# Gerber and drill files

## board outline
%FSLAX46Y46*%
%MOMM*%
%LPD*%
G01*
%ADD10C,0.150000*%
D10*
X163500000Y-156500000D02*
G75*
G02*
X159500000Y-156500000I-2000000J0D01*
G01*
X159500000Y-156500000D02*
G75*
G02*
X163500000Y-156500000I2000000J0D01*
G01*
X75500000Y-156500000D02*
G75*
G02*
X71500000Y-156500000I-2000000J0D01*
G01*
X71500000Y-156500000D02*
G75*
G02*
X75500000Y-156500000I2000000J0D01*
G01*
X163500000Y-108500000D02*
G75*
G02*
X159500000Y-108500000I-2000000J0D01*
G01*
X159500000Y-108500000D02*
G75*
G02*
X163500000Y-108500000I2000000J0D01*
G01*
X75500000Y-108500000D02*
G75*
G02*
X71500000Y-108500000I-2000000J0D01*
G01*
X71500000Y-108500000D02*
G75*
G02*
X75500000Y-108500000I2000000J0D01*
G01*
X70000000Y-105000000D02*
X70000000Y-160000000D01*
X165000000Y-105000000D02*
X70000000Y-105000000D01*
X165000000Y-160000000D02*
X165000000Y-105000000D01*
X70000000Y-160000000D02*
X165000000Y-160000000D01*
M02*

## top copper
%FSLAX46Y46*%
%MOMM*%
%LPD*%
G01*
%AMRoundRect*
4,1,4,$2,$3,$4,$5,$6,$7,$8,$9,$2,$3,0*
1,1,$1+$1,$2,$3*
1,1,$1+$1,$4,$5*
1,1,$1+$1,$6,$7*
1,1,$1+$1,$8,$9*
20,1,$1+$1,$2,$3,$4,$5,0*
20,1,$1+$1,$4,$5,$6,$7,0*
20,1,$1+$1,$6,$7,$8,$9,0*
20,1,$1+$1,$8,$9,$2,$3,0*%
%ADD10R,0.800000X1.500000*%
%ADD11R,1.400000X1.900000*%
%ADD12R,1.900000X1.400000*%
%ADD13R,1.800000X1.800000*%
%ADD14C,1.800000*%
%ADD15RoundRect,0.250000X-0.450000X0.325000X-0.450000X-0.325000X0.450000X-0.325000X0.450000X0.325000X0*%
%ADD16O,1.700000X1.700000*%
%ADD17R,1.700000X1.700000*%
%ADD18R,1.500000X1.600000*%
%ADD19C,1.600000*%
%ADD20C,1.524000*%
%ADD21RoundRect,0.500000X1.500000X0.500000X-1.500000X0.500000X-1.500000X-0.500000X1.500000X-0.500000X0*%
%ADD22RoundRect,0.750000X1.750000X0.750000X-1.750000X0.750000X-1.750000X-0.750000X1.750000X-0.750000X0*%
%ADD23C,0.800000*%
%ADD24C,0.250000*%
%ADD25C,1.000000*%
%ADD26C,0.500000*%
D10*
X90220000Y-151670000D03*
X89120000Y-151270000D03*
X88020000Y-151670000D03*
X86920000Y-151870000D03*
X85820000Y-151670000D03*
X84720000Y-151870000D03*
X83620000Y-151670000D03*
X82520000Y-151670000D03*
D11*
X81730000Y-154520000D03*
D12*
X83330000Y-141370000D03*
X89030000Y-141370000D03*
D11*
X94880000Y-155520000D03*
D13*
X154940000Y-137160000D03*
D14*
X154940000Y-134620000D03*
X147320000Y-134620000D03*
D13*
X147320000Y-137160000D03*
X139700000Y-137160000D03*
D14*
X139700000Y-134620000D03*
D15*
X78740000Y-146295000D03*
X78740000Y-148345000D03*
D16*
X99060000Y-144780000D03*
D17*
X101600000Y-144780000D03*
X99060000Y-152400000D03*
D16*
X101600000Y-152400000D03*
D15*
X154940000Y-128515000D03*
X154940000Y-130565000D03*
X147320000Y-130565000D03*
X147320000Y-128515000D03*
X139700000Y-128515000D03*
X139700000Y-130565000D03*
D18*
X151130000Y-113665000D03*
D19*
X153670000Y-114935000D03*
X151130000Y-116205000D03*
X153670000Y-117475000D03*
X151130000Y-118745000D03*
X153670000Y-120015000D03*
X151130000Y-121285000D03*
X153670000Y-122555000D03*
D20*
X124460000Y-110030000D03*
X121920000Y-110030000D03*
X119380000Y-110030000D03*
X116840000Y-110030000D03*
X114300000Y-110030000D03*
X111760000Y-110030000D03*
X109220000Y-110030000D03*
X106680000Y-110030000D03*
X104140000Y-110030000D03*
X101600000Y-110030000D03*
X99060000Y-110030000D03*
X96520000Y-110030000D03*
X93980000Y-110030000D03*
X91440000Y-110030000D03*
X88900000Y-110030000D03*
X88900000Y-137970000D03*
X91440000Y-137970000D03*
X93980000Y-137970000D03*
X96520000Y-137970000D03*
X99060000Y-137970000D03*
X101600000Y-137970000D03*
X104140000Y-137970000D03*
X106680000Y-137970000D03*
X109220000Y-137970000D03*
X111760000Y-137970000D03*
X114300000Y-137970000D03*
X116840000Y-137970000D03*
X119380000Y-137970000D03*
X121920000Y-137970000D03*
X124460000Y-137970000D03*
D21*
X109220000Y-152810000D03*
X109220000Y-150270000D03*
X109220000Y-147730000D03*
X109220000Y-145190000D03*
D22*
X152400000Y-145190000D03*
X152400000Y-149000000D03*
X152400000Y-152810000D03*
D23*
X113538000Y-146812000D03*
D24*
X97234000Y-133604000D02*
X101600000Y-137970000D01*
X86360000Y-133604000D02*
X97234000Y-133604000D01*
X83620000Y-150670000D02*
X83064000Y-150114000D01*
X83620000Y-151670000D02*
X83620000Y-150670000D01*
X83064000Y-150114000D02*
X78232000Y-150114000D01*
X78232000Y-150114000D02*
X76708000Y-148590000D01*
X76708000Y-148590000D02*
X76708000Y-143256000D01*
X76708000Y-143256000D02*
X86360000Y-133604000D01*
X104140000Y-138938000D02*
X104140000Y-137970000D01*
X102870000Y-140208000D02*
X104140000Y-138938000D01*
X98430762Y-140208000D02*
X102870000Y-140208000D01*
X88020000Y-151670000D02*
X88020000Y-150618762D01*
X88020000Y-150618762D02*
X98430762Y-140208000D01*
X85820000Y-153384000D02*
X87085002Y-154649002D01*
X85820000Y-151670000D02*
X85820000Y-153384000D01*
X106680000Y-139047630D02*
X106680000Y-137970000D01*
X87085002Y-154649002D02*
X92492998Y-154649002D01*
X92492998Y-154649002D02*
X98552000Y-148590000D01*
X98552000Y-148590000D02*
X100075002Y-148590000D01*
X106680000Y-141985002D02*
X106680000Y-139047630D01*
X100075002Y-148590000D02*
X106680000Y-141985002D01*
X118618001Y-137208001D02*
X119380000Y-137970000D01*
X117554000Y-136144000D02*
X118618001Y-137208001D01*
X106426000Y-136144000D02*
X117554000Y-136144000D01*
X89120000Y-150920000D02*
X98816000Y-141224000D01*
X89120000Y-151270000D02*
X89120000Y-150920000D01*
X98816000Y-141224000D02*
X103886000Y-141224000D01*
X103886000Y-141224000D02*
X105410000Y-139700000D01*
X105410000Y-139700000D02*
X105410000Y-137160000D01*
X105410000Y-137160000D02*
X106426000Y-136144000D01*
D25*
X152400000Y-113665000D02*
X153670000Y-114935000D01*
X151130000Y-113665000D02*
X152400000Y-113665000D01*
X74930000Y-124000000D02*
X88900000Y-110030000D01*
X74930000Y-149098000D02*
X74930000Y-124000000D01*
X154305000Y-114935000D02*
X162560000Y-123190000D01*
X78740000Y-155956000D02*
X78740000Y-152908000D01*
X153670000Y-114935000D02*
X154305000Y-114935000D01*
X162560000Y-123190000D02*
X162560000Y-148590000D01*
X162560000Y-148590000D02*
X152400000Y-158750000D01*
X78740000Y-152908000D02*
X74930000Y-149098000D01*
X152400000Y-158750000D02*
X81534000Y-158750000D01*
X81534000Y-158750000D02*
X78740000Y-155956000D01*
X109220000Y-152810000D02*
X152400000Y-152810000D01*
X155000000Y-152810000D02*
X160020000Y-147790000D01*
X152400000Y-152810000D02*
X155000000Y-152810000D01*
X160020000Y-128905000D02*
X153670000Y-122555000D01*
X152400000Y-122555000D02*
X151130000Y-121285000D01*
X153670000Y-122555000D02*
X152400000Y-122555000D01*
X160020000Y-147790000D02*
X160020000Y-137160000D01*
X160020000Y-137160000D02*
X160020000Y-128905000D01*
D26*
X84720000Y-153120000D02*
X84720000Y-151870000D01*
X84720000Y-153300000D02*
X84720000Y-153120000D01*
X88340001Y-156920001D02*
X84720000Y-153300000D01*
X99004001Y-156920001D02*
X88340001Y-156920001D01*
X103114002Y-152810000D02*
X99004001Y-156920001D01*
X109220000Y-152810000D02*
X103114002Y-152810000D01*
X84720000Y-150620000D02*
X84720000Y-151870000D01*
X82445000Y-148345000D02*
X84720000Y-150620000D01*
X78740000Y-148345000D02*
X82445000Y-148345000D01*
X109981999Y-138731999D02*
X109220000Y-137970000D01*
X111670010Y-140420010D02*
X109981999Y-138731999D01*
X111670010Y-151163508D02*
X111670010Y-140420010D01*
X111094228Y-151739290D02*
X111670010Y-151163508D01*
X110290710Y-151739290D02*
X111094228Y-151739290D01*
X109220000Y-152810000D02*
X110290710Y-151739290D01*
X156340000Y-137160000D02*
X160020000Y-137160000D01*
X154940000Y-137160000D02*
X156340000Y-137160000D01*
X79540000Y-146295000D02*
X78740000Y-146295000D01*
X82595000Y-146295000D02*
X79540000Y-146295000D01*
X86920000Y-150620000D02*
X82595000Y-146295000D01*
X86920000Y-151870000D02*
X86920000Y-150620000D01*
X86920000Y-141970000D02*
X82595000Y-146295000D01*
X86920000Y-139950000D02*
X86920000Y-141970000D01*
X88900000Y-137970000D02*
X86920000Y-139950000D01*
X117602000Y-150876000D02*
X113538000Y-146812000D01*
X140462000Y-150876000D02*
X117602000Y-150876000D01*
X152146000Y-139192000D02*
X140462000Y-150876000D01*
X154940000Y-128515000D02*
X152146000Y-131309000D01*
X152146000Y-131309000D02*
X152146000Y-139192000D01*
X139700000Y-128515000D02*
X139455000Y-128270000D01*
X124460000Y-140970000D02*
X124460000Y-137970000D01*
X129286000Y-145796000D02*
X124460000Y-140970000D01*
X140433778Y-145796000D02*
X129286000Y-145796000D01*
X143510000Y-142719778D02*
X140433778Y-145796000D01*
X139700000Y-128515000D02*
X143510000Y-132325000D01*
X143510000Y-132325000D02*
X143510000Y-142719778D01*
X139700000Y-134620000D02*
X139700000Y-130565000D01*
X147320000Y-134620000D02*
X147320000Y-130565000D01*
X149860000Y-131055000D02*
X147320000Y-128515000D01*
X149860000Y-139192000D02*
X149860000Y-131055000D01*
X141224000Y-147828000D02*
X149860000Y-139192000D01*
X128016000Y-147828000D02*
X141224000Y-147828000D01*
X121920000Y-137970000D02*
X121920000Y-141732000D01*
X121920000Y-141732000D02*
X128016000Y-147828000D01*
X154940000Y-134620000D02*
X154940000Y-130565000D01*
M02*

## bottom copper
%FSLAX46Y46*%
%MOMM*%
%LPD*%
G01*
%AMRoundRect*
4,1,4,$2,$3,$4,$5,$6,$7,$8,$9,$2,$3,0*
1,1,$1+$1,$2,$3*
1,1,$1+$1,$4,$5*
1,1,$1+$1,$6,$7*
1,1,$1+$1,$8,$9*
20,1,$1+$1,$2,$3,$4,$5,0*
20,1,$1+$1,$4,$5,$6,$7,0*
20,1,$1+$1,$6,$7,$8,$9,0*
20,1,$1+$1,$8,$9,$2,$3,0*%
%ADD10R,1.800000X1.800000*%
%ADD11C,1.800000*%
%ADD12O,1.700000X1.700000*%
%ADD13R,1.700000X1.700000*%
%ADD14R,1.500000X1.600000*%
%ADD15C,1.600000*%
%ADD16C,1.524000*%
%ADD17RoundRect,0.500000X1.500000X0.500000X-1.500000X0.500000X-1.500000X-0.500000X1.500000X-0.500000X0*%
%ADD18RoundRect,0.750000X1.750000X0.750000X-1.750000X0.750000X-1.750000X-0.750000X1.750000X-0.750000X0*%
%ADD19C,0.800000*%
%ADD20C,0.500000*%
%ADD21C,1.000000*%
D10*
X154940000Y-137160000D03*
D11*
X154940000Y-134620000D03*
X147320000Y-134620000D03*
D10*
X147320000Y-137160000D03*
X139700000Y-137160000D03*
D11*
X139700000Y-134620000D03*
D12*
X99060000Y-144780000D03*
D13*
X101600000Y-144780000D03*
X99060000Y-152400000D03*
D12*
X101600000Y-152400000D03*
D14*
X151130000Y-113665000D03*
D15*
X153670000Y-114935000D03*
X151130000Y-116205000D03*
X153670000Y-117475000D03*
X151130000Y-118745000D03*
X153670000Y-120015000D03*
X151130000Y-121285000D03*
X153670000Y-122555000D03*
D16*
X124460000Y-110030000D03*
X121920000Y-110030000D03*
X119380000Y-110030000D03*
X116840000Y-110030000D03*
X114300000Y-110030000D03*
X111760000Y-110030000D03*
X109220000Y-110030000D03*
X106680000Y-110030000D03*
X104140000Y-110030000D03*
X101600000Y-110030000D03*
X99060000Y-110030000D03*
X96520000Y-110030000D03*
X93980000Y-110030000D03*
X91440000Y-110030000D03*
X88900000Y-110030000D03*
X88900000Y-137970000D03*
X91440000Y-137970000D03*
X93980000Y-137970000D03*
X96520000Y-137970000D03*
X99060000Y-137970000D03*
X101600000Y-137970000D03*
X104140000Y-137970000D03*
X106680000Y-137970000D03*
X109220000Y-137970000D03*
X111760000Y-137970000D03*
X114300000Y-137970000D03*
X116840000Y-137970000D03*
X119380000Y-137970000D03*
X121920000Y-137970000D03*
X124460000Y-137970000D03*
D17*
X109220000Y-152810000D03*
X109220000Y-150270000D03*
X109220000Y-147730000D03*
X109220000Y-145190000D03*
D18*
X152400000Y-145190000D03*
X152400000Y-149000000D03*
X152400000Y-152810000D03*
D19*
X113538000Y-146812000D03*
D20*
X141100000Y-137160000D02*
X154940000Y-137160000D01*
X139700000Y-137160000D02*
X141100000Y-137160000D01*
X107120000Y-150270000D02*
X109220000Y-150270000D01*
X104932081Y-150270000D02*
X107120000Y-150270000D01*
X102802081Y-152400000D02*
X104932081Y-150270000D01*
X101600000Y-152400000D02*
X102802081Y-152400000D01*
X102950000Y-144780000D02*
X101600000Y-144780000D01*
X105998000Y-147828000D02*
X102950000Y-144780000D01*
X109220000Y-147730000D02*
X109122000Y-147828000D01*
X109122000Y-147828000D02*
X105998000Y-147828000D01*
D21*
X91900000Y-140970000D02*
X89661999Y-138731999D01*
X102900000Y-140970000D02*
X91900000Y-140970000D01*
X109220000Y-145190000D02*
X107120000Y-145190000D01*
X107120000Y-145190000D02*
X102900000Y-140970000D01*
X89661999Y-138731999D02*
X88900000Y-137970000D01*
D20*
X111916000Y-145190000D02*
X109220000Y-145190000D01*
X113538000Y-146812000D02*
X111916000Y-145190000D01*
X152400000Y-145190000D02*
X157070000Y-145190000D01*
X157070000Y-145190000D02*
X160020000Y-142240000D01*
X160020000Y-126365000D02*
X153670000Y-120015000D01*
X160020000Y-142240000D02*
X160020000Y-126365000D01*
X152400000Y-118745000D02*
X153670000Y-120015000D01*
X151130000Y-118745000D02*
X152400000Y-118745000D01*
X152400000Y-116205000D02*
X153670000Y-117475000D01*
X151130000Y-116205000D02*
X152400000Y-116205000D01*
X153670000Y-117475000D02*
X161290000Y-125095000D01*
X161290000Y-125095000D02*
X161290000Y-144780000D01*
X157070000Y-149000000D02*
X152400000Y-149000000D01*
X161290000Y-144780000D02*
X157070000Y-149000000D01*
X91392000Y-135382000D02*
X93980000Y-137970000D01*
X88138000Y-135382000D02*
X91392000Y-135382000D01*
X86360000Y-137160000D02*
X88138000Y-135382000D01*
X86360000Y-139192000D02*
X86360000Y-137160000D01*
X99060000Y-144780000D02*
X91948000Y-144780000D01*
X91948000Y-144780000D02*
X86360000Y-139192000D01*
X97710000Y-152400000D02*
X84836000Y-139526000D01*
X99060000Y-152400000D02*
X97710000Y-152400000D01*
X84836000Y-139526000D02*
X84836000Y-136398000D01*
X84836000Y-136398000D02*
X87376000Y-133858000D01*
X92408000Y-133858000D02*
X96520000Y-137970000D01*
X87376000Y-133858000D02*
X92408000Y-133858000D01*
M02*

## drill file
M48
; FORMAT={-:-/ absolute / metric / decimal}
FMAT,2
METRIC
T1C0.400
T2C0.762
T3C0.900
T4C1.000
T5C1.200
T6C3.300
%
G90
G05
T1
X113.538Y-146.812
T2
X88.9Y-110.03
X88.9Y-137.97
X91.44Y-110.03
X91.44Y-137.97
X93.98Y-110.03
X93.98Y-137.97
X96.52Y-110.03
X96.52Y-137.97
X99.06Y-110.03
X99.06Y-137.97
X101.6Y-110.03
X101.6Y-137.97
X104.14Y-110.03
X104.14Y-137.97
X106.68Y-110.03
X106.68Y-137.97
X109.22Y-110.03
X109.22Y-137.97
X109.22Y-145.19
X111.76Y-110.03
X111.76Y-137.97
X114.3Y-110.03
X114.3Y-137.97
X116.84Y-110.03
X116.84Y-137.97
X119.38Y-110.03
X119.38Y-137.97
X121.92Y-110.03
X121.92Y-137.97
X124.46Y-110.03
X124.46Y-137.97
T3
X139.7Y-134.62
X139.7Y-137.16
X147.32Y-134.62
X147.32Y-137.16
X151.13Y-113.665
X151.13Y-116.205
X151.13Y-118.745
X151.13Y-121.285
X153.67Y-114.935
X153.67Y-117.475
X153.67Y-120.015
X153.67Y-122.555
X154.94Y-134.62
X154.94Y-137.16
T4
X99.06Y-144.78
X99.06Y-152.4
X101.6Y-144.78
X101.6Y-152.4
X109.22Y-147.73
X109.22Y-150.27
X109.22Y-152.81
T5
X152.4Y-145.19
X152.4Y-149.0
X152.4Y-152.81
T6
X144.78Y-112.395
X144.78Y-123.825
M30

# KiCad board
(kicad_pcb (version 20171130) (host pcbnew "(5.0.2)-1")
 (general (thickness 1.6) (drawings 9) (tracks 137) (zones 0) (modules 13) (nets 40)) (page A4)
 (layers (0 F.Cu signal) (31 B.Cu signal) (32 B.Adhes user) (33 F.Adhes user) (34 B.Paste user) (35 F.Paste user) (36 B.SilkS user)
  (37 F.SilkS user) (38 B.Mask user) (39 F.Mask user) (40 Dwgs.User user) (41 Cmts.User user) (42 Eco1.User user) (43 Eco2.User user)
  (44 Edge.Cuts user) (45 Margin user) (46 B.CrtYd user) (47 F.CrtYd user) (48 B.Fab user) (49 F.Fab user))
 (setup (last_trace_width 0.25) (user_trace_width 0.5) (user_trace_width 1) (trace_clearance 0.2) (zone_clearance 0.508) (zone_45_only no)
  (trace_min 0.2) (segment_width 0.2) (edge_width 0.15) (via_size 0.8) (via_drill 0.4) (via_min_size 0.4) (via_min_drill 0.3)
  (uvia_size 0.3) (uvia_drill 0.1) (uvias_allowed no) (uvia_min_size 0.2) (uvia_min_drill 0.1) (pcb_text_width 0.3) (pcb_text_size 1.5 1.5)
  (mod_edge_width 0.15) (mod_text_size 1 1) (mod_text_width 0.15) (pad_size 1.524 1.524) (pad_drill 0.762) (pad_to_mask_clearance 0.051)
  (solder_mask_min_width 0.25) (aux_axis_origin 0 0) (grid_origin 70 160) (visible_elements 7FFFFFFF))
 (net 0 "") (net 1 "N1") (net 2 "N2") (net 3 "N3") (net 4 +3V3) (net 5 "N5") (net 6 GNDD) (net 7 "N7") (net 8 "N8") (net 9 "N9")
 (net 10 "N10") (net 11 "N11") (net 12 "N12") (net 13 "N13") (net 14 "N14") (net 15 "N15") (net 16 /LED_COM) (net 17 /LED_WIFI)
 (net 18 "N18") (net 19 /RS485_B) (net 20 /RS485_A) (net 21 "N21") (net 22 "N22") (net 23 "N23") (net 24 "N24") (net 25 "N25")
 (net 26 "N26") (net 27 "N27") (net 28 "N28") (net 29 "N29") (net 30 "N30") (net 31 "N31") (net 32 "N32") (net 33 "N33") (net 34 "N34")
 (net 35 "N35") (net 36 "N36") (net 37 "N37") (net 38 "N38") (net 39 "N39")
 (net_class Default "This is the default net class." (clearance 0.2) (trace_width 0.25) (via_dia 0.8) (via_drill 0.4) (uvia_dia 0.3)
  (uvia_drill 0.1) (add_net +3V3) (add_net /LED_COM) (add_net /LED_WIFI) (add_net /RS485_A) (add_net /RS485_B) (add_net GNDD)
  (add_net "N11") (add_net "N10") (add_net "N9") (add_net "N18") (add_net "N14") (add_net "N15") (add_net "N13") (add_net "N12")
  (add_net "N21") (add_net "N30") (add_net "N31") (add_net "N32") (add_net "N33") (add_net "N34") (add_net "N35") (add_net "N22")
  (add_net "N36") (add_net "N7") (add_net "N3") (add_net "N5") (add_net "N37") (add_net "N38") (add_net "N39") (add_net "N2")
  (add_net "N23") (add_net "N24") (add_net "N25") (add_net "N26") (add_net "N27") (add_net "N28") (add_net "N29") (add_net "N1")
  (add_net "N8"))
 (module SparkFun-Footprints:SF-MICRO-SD (layer F.Cu) (at 81.28 140.97 180)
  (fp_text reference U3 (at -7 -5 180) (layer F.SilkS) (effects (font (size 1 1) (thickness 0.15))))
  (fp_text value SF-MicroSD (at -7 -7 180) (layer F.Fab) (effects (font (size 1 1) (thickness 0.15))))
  (pad 1 smd rect (at -8.94 -10.7 270) (size 1.5 0.8) (layers F.Cu F.Paste F.Mask) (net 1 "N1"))
  (pad 2 smd rect (at -7.84 -10.3 270) (size 1.5 0.8) (layers F.Cu F.Paste F.Mask) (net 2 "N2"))
  (pad 3 smd rect (at -6.74 -10.7 270) (size 1.5 0.8) (layers F.Cu F.Paste F.Mask) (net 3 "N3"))
  (pad 4 smd rect (at -5.64 -10.9 270) (size 1.5 0.8) (layers F.Cu F.Paste F.Mask) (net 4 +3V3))
  (pad 5 smd rect (at -4.54 -10.7 270) (size 1.5 0.8) (layers F.Cu F.Paste F.Mask) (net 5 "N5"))
  (pad 6 smd rect (at -3.44 -10.9 270) (size 1.5 0.8) (layers F.Cu F.Paste F.Mask) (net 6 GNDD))
  (pad 7 smd rect (at -2.34 -10.7 270) (size 1.5 0.8) (layers F.Cu F.Paste F.Mask) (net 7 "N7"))
  (pad 8 smd rect (at -1.24 -10.7 270) (size 1.5 0.8) (layers F.Cu F.Paste F.Mask) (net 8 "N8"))
  (pad 9 smd rect (at -0.45 -13.55 270) (size 1.9 1.4) (layers F.Cu F.Paste F.Mask))
  (pad 10 smd rect (at -2.05 -0.4 180) (size 1.9 1.4) (layers F.Cu F.Paste F.Mask))
  (pad 11 smd rect (at -7.75 -0.4 180) (size 1.9 1.4) (layers F.Cu F.Paste F.Mask))
  (pad 12 smd rect (at -13.6 -14.55 270) (size 1.9 1.4) (layers F.Cu F.Paste F.Mask)))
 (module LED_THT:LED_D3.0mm (layer F.Cu) (at 154.94 137.16 90)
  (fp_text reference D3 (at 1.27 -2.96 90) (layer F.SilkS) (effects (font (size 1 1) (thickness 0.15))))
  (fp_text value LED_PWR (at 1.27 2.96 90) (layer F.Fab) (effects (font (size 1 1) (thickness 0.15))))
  (pad 1 thru_hole rect (at 0 0 90) (size 1.8 1.8) (drill 0.9) (layers *.Cu *.Mask) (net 6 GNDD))
  (pad 2 thru_hole circle (at 2.54 0 90) (size 1.8 1.8) (drill 0.9) (layers *.Cu *.Mask) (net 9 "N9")))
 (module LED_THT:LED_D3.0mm (layer F.Cu) (at 147.32 137.16 90)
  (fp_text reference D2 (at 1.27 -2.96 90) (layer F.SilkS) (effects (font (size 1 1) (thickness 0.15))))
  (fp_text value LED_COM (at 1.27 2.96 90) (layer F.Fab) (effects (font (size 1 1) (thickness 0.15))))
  (pad 2 thru_hole circle (at 2.54 0 90) (size 1.8 1.8) (drill 0.9) (layers *.Cu *.Mask) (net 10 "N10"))
  (pad 1 thru_hole rect (at 0 0 90) (size 1.8 1.8) (drill 0.9) (layers *.Cu *.Mask) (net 6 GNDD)))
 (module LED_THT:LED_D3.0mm (layer F.Cu) (at 139.7 137.16 90)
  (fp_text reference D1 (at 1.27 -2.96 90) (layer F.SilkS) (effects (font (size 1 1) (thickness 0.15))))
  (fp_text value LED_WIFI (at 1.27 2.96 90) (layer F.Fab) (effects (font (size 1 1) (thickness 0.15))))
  (pad 1 thru_hole rect (at 0 0 90) (size 1.8 1.8) (drill 0.9) (layers *.Cu *.Mask) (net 6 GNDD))
  (pad 2 thru_hole circle (at 2.54 0 90) (size 1.8 1.8) (drill 0.9) (layers *.Cu *.Mask) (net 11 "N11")))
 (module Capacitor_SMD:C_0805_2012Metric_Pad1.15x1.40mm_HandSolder (layer F.Cu) (at 78.74 147.32 270)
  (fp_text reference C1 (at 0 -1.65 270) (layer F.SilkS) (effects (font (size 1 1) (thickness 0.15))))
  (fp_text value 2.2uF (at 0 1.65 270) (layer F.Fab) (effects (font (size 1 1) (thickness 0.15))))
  (pad 1 smd roundrect (at -1.025 0 270) (size 1.15 1.4) (layers F.Cu F.Paste F.Mask) (roundrect_rratio 0.217391) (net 4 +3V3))
  (pad 2 smd roundrect (at 1.025 0 270) (size 1.15 1.4) (layers F.Cu F.Paste F.Mask) (roundrect_rratio 0.217391) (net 6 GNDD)))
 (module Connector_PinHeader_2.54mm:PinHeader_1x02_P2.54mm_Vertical (layer F.Cu) (at 101.6 144.78 270)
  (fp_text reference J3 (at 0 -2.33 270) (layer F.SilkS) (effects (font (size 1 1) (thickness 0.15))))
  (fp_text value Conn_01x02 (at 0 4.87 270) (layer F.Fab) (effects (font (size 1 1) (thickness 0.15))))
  (pad 2 thru_hole oval (at 0 2.54 270) (size 1.7 1.7) (drill 1) (layers *.Cu *.Mask) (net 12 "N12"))
  (pad 1 thru_hole rect (at 0 0 270) (size 1.7 1.7) (drill 1) (layers *.Cu *.Mask) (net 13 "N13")))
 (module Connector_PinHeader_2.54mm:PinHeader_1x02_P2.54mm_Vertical (layer F.Cu) (at 99.06 152.4 90)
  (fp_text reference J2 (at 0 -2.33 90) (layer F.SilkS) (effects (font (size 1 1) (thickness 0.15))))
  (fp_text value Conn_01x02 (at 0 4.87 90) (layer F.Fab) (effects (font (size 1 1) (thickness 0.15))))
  (pad 1 thru_hole rect (at 0 0 90) (size 1.7 1.7) (drill 1) (layers *.Cu *.Mask) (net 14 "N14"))
  (pad 2 thru_hole oval (at 0 2.54 90) (size 1.7 1.7) (drill 1) (layers *.Cu *.Mask) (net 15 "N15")))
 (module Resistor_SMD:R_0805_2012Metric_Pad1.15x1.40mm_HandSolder (layer F.Cu) (at 154.94 129.54 270)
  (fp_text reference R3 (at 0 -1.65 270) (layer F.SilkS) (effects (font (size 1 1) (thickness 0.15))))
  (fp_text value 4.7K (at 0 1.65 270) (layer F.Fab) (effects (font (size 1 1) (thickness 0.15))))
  (pad 1 smd roundrect (at -1.025 0 270) (size 1.15 1.4) (layers F.Cu F.Paste F.Mask) (roundrect_rratio 0.217391) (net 4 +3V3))
  (pad 2 smd roundrect (at 1.025 0 270) (size 1.15 1.4) (layers F.Cu F.Paste F.Mask) (roundrect_rratio 0.217391) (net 9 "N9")))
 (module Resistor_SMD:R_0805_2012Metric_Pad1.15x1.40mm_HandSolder (layer F.Cu) (at 147.32 129.54 270)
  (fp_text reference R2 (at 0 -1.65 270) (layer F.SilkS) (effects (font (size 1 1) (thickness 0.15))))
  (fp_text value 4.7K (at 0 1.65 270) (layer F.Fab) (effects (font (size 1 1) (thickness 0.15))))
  (pad 2 smd roundrect (at 1.025 0 270) (size 1.15 1.4) (layers F.Cu F.Paste F.Mask) (roundrect_rratio 0.217391) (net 10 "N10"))
  (pad 1 smd roundrect (at -1.025 0 270) (size 1.15 1.4) (layers F.Cu F.Paste F.Mask) (roundrect_rratio 0.217391) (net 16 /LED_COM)))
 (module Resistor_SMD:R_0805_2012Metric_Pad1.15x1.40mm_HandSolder (layer F.Cu) (at 139.7 129.54 270)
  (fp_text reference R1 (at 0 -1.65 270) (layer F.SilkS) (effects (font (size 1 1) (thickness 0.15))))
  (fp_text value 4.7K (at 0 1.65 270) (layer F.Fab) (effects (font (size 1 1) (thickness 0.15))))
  (pad 1 smd roundrect (at -1.025 0 270) (size 1.15 1.4) (layers F.Cu F.Paste F.Mask) (roundrect_rratio 0.217391) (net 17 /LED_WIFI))
  (pad 2 smd roundrect (at 1.025 0 270) (size 1.15 1.4) (layers F.Cu F.Paste F.Mask) (roundrect_rratio 0.217391) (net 11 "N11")))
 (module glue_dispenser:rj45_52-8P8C (layer F.Cu) (at 153.67 118.11 270)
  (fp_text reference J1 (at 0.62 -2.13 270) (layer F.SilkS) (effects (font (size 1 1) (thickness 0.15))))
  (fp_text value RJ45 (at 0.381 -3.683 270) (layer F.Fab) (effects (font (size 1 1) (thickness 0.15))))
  (pad "" np_thru_hole circle (at -5.715 8.89 270) (size 3.3 3.3) (drill 3.3) (layers *.Cu *.Mask))
  (pad "" np_thru_hole circle (at 5.715 8.89 270) (size 3.3 3.3) (drill 3.3) (layers *.Cu *.Mask))
  (pad 1 thru_hole rect (at -4.445 2.54 270) (size 1.6 1.5) (drill 0.9) (layers *.Cu *.Mask) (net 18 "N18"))
  (pad 2 thru_hole circle (at -3.175 0 270) (size 1.6 1.6) (drill 0.9) (layers *.Cu *.Mask) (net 18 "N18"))
  (pad 3 thru_hole circle (at -1.905 2.54 270) (size 1.6 1.6) (drill 0.9) (layers *.Cu *.Mask) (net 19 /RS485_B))
  (pad 4 thru_hole circle (at -0.635 0 270) (size 1.6 1.6) (drill 0.9) (layers *.Cu *.Mask) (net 19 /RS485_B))
  (pad 5 thru_hole circle (at 0.635 2.54 270) (size 1.6 1.6) (drill 0.9) (layers *.Cu *.Mask) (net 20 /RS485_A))
  (pad 6 thru_hole circle (at 1.905 0 270) (size 1.6 1.6) (drill 0.9) (layers *.Cu *.Mask) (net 20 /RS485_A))
  (pad 7 thru_hole circle (at 3.175 2.54 270) (size 1.6 1.6) (drill 0.9) (layers *.Cu *.Mask) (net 6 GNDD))
  (pad 8 thru_hole circle (at 4.445 0 270) (size 1.6 1.6) (drill 0.9) (layers *.Cu *.Mask) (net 6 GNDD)))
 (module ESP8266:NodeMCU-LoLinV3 (layer F.Cu) (at 104.14 124 270)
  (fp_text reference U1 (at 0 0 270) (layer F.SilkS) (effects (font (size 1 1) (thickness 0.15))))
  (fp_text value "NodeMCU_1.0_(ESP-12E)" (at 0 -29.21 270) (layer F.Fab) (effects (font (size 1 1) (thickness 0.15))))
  (pad 1 thru_hole circle (at -13.97 -20.32 270) (size 1.524 1.524) (drill 0.762) (layers *.Cu *.Mask F.SilkS) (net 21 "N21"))
  (pad 2 thru_hole circle (at -13.97 -17.78 270) (size 1.524 1.524) (drill 0.762) (layers *.Cu *.Mask F.SilkS) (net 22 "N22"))
  (pad 3 thru_hole circle (at -13.97 -15.24 270) (size 1.524 1.524) (drill 0.762) (layers *.Cu *.Mask F.SilkS) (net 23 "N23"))
  (pad 4 thru_hole circle (at -13.97 -12.7 270) (size 1.524 1.524) (drill 0.762) (layers *.Cu *.Mask F.SilkS) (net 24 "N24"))
  (pad 5 thru_hole circle (at -13.97 -10.16 270) (size 1.524 1.524) (drill 0.762) (layers *.Cu *.Mask F.SilkS) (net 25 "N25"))
  (pad 6 thru_hole circle (at -13.97 -7.62 270) (size 1.524 1.524) (drill 0.762) (layers *.Cu *.Mask F.SilkS) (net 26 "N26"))
  (pad 7 thru_hole circle (at -13.97 -5.08 270) (size 1.524 1.524) (drill 0.762) (layers *.Cu *.Mask F.SilkS) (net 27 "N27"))
  (pad 8 thru_hole circle (at -13.97 -2.54 270) (size 1.524 1.524) (drill 0.762) (layers *.Cu *.Mask F.SilkS) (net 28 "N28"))
  (pad 9 thru_hole circle (at -13.97 0 270) (size 1.524 1.524) (drill 0.762) (layers *.Cu *.Mask F.SilkS) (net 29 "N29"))
  (pad 10 thru_hole circle (at -13.97 2.54 270) (size 1.524 1.524) (drill 0.762) (layers *.Cu *.Mask F.SilkS) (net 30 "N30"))
  (pad 11 thru_hole circle (at -13.97 5.08 270) (size 1.524 1.524) (drill 0.762) (layers *.Cu *.Mask F.SilkS) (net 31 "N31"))
  (pad 12 thru_hole circle (at -13.97 7.62 270) (size 1.524 1.524) (drill 0.762) (layers *.Cu *.Mask F.SilkS) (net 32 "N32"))
  (pad 13 thru_hole circle (at -13.97 10.16 270) (size 1.524 1.524) (drill 0.762) (layers *.Cu *.Mask F.SilkS) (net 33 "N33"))
  (pad 14 thru_hole circle (at -13.97 12.7 270) (size 1.524 1.524) (drill 0.762) (layers *.Cu *.Mask F.SilkS) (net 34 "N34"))
  (pad 15 thru_hole circle (at -13.97 15.24 270) (size 1.524 1.524) (drill 0.762) (layers *.Cu *.Mask F.SilkS) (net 18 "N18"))
  (pad 16 thru_hole circle (at 13.97 15.24 270) (size 1.524 1.524) (drill 0.762) (layers *.Cu *.Mask F.SilkS) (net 4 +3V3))
  (pad 17 thru_hole circle (at 13.97 12.7 270) (size 1.524 1.524) (drill 0.762) (layers *.Cu *.Mask F.SilkS) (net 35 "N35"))
  (pad 18 thru_hole circle (at 13.97 10.16 270) (size 1.524 1.524) (drill 0.762) (layers *.Cu *.Mask F.SilkS) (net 12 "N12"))
  (pad 19 thru_hole circle (at 13.97 7.62 270) (size 1.524 1.524) (drill 0.762) (layers *.Cu *.Mask F.SilkS) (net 14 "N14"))
  (pad 20 thru_hole circle (at 13.97 5.08 270) (size 1.524 1.524) (drill 0.762) (layers *.Cu *.Mask F.SilkS) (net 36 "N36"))
  (pad 21 thru_hole circle (at 13.97 2.54 270) (size 1.524 1.524) (drill 0.762) (layers *.Cu *.Mask F.SilkS) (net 7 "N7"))
  (pad 22 thru_hole circle (at 13.97 0 270) (size 1.524 1.524) (drill 0.762) (layers *.Cu *.Mask F.SilkS) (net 3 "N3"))
  (pad 23 thru_hole circle (at 13.97 -2.54 270) (size 1.524 1.524) (drill 0.762) (layers *.Cu *.Mask F.SilkS) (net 5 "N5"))
  (pad 24 thru_hole circle (at 13.97 -5.08 270) (size 1.524 1.524) (drill 0.762) (layers *.Cu *.Mask F.SilkS) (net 6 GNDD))
  (pad 25 thru_hole circle (at 13.97 -7.62 270) (size 1.524 1.524) (drill 0.762) (layers *.Cu *.Mask F.SilkS) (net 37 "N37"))
  (pad 26 thru_hole circle (at 13.97 -10.16 270) (size 1.524 1.524) (drill 0.762) (layers *.Cu *.Mask F.SilkS) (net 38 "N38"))
  (pad 27 thru_hole circle (at 13.97 -12.7 270) (size 1.524 1.524) (drill 0.762) (layers *.Cu *.Mask F.SilkS) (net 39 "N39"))
  (pad 28 thru_hole circle (at 13.97 -15.24 270) (size 1.524 1.524) (drill 0.762) (layers *.Cu *.Mask F.SilkS) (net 2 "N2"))
  (pad 29 thru_hole circle (at 13.97 -17.78 270) (size 1.524 1.524) (drill 0.762) (layers *.Cu *.Mask F.SilkS) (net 16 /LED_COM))
  (pad 30 thru_hole circle (at 13.97 -20.32 270) (size 1.524 1.524) (drill 0.762) (layers *.Cu *.Mask F.SilkS) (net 17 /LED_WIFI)))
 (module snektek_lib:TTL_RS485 (layer F.Cu) (at 152.4 149 180)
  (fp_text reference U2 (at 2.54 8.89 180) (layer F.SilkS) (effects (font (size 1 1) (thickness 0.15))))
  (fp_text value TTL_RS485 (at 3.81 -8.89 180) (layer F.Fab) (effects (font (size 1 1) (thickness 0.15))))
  (pad 1 thru_hole roundrect (at 43.18 -3.81 180) (size 4 2) (drill 1) (layers *.Cu *.Mask) (roundrect_rratio 0.25) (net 6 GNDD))
  (pad 2 thru_hole roundrect (at 43.18 -1.27 180) (size 4 2) (drill 1) (layers *.Cu *.Mask) (roundrect_rratio 0.25) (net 15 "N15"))
  (pad 3 thru_hole roundrect (at 43.18 1.27 180) (size 4 2) (drill 1) (layers *.Cu *.Mask) (roundrect_rratio 0.25) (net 13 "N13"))
  (pad 4 thru_hole roundrect (at 43.18 3.81 180) (size 4 2) (drill 0.762) (layers *.Cu *.Mask) (roundrect_rratio 0.25) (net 4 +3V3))
  (pad 5 thru_hole roundrect (at 0 3.81 180) (size 5 3) (drill 1.2) (layers *.Cu *.Mask) (roundrect_rratio 0.25) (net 20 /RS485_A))
  (pad 6 thru_hole roundrect (at 0 0 180) (size 5 3) (drill 1.2) (layers *.Cu *.Mask) (roundrect_rratio 0.25) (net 19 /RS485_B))
  (pad 7 thru_hole roundrect (at 0 -3.81 180) (size 5 3) (drill 1.2) (layers *.Cu *.Mask) (roundrect_rratio 0.25) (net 6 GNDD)))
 (gr_circle (center 161.5 156.5) (end 163.5 156.5) (layer Edge.Cuts) (width 0.15))
 (gr_circle (center 73.5 156.5) (end 75.5 156.5) (layer Edge.Cuts) (width 0.15))
 (gr_circle (center 161.5 108.5) (end 163.5 108.5) (layer Edge.Cuts) (width 0.15))
 (gr_circle (center 73.5 108.5) (end 75.5 108.5) (layer Edge.Cuts) (width 0.15))
 (gr_line (start 70 105) (end 70 160) (layer Edge.Cuts) (width 0.15))
 (gr_line (start 165 105) (end 70 105) (layer Edge.Cuts) (width 0.15))
 (gr_line (start 165 160) (end 165 105) (layer Edge.Cuts) (width 0.15))
 (gr_line (start 70 160) (end 165 160) (layer Edge.Cuts) (width 0.15))
 (segment (start 97.234 133.604) (end 101.6 137.97) (width 0.25) (layer F.Cu) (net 7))
 (segment (start 86.36 133.604) (end 97.234 133.604) (width 0.25) (layer F.Cu) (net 7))
 (segment (start 83.62 150.67) (end 83.064 150.114) (width 0.25) (layer F.Cu) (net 7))
 (segment (start 83.62 151.67) (end 83.62 150.67) (width 0.25) (layer F.Cu) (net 7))
 (segment (start 83.064 150.114) (end 78.232 150.114) (width 0.25) (layer F.Cu) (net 7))
 (segment (start 78.232 150.114) (end 76.708 148.59) (width 0.25) (layer F.Cu) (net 7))
 (segment (start 76.708 148.59) (end 76.708 143.256) (width 0.25) (layer F.Cu) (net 7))
 (segment (start 76.708 143.256) (end 86.36 133.604) (width 0.25) (layer F.Cu) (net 7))
 (segment (start 104.14 138.938) (end 104.14 137.97) (width 0.25) (layer F.Cu) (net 3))
 (segment (start 102.87 140.208) (end 104.14 138.938) (width 0.25) (layer F.Cu) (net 3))
 (segment (start 98.430762 140.208) (end 102.87 140.208) (width 0.25) (layer F.Cu) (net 3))
 (segment (start 88.02 151.67) (end 88.02 150.618762) (width 0.25) (layer F.Cu) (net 3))
 (segment (start 88.02 150.618762) (end 98.430762 140.208) (width 0.25) (layer F.Cu) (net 3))
 (segment (start 85.82 153.384) (end 87.085002 154.649002) (width 0.25) (layer F.Cu) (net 5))
 (segment (start 85.82 151.67) (end 85.82 153.384) (width 0.25) (layer F.Cu) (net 5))
 (segment (start 106.68 139.04763) (end 106.68 137.97) (width 0.25) (layer F.Cu) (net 5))
 (segment (start 87.085002 154.649002) (end 92.492998 154.649002) (width 0.25) (layer F.Cu) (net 5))
 (segment (start 92.492998 154.649002) (end 98.552 148.59) (width 0.25) (layer F.Cu) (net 5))
 (segment (start 98.552 148.59) (end 100.075002 148.59) (width 0.25) (layer F.Cu) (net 5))
 (segment (start 106.68 141.985002) (end 106.68 139.04763) (width 0.25) (layer F.Cu) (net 5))
 (segment (start 100.075002 148.59) (end 106.68 141.985002) (width 0.25) (layer F.Cu) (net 5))
 (segment (start 118.618001 137.208001) (end 119.38 137.97) (width 0.25) (layer F.Cu) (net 2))
 (segment (start 117.554 136.144) (end 118.618001 137.208001) (width 0.25) (layer F.Cu) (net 2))
 (segment (start 106.426 136.144) (end 117.554 136.144) (width 0.25) (layer F.Cu) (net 2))
 (segment (start 89.12 150.92) (end 98.816 141.224) (width 0.25) (layer F.Cu) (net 2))
 (segment (start 89.12 151.27) (end 89.12 150.92) (width 0.25) (layer F.Cu) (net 2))
 (segment (start 98.816 141.224) (end 103.886 141.224) (width 0.25) (layer F.Cu) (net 2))
 (segment (start 103.886 141.224) (end 105.41 139.7) (width 0.25) (layer F.Cu) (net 2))
 (segment (start 105.41 139.7) (end 105.41 137.16) (width 0.25) (layer F.Cu) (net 2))
 (segment (start 105.41 137.16) (end 106.426 136.144) (width 0.25) (layer F.Cu) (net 2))
 (segment (start 152.4 113.665) (end 153.67 114.935) (width 1) (layer F.Cu) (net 18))
 (segment (start 151.13 113.665) (end 152.4 113.665) (width 1) (layer F.Cu) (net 18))
 (segment (start 74.93 124) (end 88.9 110.03) (width 1) (layer F.Cu) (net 18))
 (segment (start 74.93 149.098) (end 74.93 124) (width 1) (layer F.Cu) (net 18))
 (segment (start 154.305 114.935) (end 162.56 123.19) (width 1) (layer F.Cu) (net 18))
 (segment (start 78.74 155.956) (end 78.74 152.908) (width 1) (layer F.Cu) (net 18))
 (segment (start 153.67 114.935) (end 154.305 114.935) (width 1) (layer F.Cu) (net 18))
 (segment (start 162.56 123.19) (end 162.56 148.59) (width 1) (layer F.Cu) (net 18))
 (segment (start 162.56 148.59) (end 152.4 158.75) (width 1) (layer F.Cu) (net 18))
 (segment (start 78.74 152.908) (end 74.93 149.098) (width 1) (layer F.Cu) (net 18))
 (segment (start 152.4 158.75) (end 81.534 158.75) (width 1) (layer F.Cu) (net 18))
 (segment (start 81.534 158.75) (end 78.74 155.956) (width 1) (layer F.Cu) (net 18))
 (segment (start 109.22 152.81) (end 152.4 152.81) (width 1) (layer F.Cu) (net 6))
 (segment (start 155 152.81) (end 160.02 147.79) (width 1) (layer F.Cu) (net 6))
 (segment (start 152.4 152.81) (end 155 152.81) (width 1) (layer F.Cu) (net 6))
 (segment (start 160.02 128.905) (end 153.67 122.555) (width 1) (layer F.Cu) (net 6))
 (segment (start 152.4 122.555) (end 151.13 121.285) (width 1) (layer F.Cu) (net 6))
 (segment (start 153.67 122.555) (end 152.4 122.555) (width 1) (layer F.Cu) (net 6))
 (segment (start 160.02 147.79) (end 160.02 137.16) (width 1) (layer F.Cu) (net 6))
 (segment (start 160.02 137.16) (end 160.02 128.905) (width 1) (layer F.Cu) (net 6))
 (segment (start 84.72 153.12) (end 84.72 151.87) (width 0.5) (layer F.Cu) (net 6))
 (segment (start 84.72 153.3) (end 84.72 153.12) (width 0.5) (layer F.Cu) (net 6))
 (segment (start 88.340001 156.920001) (end 84.72 153.3) (width 0.5) (layer F.Cu) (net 6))
 (segment (start 99.004001 156.920001) (end 88.340001 156.920001) (width 0.5) (layer F.Cu) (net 6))
 (segment (start 103.114002 152.81) (end 99.004001 156.920001) (width 0.5) (layer F.Cu) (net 6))
 (segment (start 109.22 152.81) (end 103.114002 152.81) (width 0.5) (layer F.Cu) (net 6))
 (segment (start 84.72 150.62) (end 84.72 151.87) (width 0.5) (layer F.Cu) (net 6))
 (segment (start 82.445 148.345) (end 84.72 150.62) (width 0.5) (layer F.Cu) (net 6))
 (segment (start 78.74 148.345) (end 82.445 148.345) (width 0.5) (layer F.Cu) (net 6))
 (segment (start 109.981999 138.731999) (end 109.22 137.97) (width 0.5) (layer F.Cu) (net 6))
 (segment (start 111.67001 140.42001) (end 109.981999 138.731999) (width 0.5) (layer F.Cu) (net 6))
 (segment (start 111.67001 151.163508) (end 111.67001 140.42001) (width 0.5) (layer F.Cu) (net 6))
 (segment (start 111.094228 151.73929) (end 111.67001 151.163508) (width 0.5) (layer F.Cu) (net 6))
 (segment (start 110.29071 151.73929) (end 111.094228 151.73929) (width 0.5) (layer F.Cu) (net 6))
 (segment (start 109.22 152.81) (end 110.29071 151.73929) (width 0.5) (layer F.Cu) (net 6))
 (segment (start 156.34 137.16) (end 160.02 137.16) (width 0.5) (layer F.Cu) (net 6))
 (segment (start 154.94 137.16) (end 156.34 137.16) (width 0.5) (layer F.Cu) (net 6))
 (segment (start 141.1 137.16) (end 154.94 137.16) (width 0.5) (layer B.Cu) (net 6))
 (segment (start 139.7 137.16) (end 141.1 137.16) (width 0.5) (layer B.Cu) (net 6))
 (segment (start 107.12 150.27) (end 109.22 150.27) (width 0.5) (layer B.Cu) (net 15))
 (segment (start 104.932081 150.27) (end 107.12 150.27) (width 0.5) (layer B.Cu) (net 15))
 (segment (start 102.802081 152.4) (end 104.932081 150.27) (width 0.5) (layer B.Cu) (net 15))
 (segment (start 101.6 152.4) (end 102.802081 152.4) (width 0.5) (layer B.Cu) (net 15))
 (segment (start 102.95 144.78) (end 101.6 144.78) (width 0.5) (layer B.Cu) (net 13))
 (segment (start 105.998 147.828) (end 102.95 144.78) (width 0.5) (layer B.Cu) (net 13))
 (segment (start 109.22 147.73) (end 109.122 147.828) (width 0.5) (layer B.Cu) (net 13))
 (segment (start 109.122 147.828) (end 105.998 147.828) (width 0.5) (layer B.Cu) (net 13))
 (segment (start 91.9 140.97) (end 89.661999 138.731999) (width 1) (layer B.Cu) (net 4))
 (segment (start 102.9 140.97) (end 91.9 140.97) (width 1) (layer B.Cu) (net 4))
 (segment (start 109.22 145.19) (end 107.12 145.19) (width 1) (layer B.Cu) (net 4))
 (segment (start 107.12 145.19) (end 102.9 140.97) (width 1) (layer B.Cu) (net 4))
 (segment (start 89.661999 138.731999) (end 88.9 137.97) (width 1) (layer B.Cu) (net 4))
 (segment (start 79.54 146.295) (end 78.74 146.295) (width 0.5) (layer F.Cu) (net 4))
 (segment (start 82.595 146.295) (end 79.54 146.295) (width 0.5) (layer F.Cu) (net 4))
 (segment (start 86.92 150.62) (end 82.595 146.295) (width 0.5) (layer F.Cu) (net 4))
 (segment (start 86.92 151.87) (end 86.92 150.62) (width 0.5) (layer F.Cu) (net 4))
 (segment (start 111.916 145.19) (end 109.22 145.19) (width 0.5) (layer B.Cu) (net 4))
 (segment (start 113.538 146.812) (end 111.916 145.19) (width 0.5) (layer B.Cu) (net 4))
 (via (at 113.538 146.812) (size 0.8) (drill 0.4) (layers F.Cu B.Cu) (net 4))
 (segment (start 86.92 141.97) (end 82.595 146.295) (width 0.5) (layer F.Cu) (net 4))
 (segment (start 86.92 139.95) (end 86.92 141.97) (width 0.5) (layer F.Cu) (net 4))
 (segment (start 88.9 137.97) (end 86.92 139.95) (width 0.5) (layer F.Cu) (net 4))
 (segment (start 117.602 150.876) (end 113.538 146.812) (width 0.5) (layer F.Cu) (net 4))
 (segment (start 140.462 150.876) (end 117.602 150.876) (width 0.5) (layer F.Cu) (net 4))
 (segment (start 152.146 139.192) (end 140.462 150.876) (width 0.5) (layer F.Cu) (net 4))
 (segment (start 154.94 128.515) (end 152.146 131.309) (width 0.5) (layer F.Cu) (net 4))
 (segment (start 152.146 131.309) (end 152.146 139.192) (width 0.5) (layer F.Cu) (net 4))
 (segment (start 152.4 145.19) (end 157.07 145.19) (width 0.5) (layer B.Cu) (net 20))
 (segment (start 157.07 145.19) (end 160.02 142.24) (width 0.5) (layer B.Cu) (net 20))
 (segment (start 160.02 126.365) (end 153.67 120.015) (width 0.5) (layer B.Cu) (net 20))
 (segment (start 160.02 142.24) (end 160.02 126.365) (width 0.5) (layer B.Cu) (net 20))
 (segment (start 152.4 118.745) (end 153.67 120.015) (width 0.5) (layer B.Cu) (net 20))
 (segment (start 151.13 118.745) (end 152.4 118.745) (width 0.5) (layer B.Cu) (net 20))
 (segment (start 152.4 116.205) (end 153.67 117.475) (width 0.5) (layer B.Cu) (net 19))
 (segment (start 151.13 116.205) (end 152.4 116.205) (width 0.5) (layer B.Cu) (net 19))
 (segment (start 153.67 117.475) (end 161.29 125.095) (width 0.5) (layer B.Cu) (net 19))
 (segment (start 161.29 125.095) (end 161.29 144.78) (width 0.5) (layer B.Cu) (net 19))
 (segment (start 157.07 149) (end 152.4 149) (width 0.5) (layer B.Cu) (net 19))
 (segment (start 161.29 144.78) (end 157.07 149) (width 0.5) (layer B.Cu) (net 19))
 (segment (start 91.392 135.382) (end 93.98 137.97) (width 0.5) (layer B.Cu) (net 12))
 (segment (start 88.138 135.382) (end 91.392 135.382) (width 0.5) (layer B.Cu) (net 12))
 (segment (start 86.36 137.16) (end 88.138 135.382) (width 0.5) (layer B.Cu) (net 12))
 (segment (start 86.36 139.192) (end 86.36 137.16) (width 0.5) (layer B.Cu) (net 12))
 (segment (start 99.06 144.78) (end 91.948 144.78) (width 0.5) (layer B.Cu) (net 12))
 (segment (start 91.948 144.78) (end 86.36 139.192) (width 0.5) (layer B.Cu) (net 12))
 (segment (start 97.71 152.4) (end 84.836 139.526) (width 0.5) (layer B.Cu) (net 14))
 (segment (start 99.06 152.4) (end 97.71 152.4) (width 0.5) (layer B.Cu) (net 14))
 (segment (start 84.836 139.526) (end 84.836 136.398) (width 0.5) (layer B.Cu) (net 14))
 (segment (start 84.836 136.398) (end 87.376 133.858) (width 0.5) (layer B.Cu) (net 14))
 (segment (start 92.408 133.858) (end 96.52 137.97) (width 0.5) (layer B.Cu) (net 14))
 (segment (start 87.376 133.858) (end 92.408 133.858) (width 0.5) (layer B.Cu) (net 14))
 (segment (start 139.7 128.515) (end 139.455 128.27) (width 0.5) (layer F.Cu) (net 17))
 (segment (start 124.46 140.97) (end 124.46 137.97) (width 0.5) (layer F.Cu) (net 17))
 (segment (start 129.286 145.796) (end 124.46 140.97) (width 0.5) (layer F.Cu) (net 17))
 (segment (start 140.433778 145.796) (end 129.286 145.796) (width 0.5) (layer F.Cu) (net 17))
 (segment (start 143.51 142.719778) (end 140.433778 145.796) (width 0.5) (layer F.Cu) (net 17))
 (segment (start 139.7 128.515) (end 143.51 132.325) (width 0.5) (layer F.Cu) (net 17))
 (segment (start 143.51 132.325) (end 143.51 142.719778) (width 0.5) (layer F.Cu) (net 17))
 (segment (start 139.7 134.62) (end 139.7 130.565) (width 0.5) (layer F.Cu) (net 11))
 (segment (start 147.32 134.62) (end 147.32 130.565) (width 0.5) (layer F.Cu) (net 10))
 (segment (start 149.86 131.055) (end 147.32 128.515) (width 0.5) (layer F.Cu) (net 16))
 (segment (start 149.86 139.192) (end 149.86 131.055) (width 0.5) (layer F.Cu) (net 16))
 (segment (start 141.224 147.828) (end 149.86 139.192) (width 0.5) (layer F.Cu) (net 16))
 (segment (start 128.016 147.828) (end 141.224 147.828) (width 0.5) (layer F.Cu) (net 16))
 (segment (start 121.92 137.97) (end 121.92 141.732) (width 0.5) (layer F.Cu) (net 16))
 (segment (start 121.92 141.732) (end 128.016 147.828) (width 0.5) (layer F.Cu) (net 16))
 (segment (start 154.94 134.62) (end 154.94 130.565) (width 0.5) (layer F.Cu) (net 9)))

